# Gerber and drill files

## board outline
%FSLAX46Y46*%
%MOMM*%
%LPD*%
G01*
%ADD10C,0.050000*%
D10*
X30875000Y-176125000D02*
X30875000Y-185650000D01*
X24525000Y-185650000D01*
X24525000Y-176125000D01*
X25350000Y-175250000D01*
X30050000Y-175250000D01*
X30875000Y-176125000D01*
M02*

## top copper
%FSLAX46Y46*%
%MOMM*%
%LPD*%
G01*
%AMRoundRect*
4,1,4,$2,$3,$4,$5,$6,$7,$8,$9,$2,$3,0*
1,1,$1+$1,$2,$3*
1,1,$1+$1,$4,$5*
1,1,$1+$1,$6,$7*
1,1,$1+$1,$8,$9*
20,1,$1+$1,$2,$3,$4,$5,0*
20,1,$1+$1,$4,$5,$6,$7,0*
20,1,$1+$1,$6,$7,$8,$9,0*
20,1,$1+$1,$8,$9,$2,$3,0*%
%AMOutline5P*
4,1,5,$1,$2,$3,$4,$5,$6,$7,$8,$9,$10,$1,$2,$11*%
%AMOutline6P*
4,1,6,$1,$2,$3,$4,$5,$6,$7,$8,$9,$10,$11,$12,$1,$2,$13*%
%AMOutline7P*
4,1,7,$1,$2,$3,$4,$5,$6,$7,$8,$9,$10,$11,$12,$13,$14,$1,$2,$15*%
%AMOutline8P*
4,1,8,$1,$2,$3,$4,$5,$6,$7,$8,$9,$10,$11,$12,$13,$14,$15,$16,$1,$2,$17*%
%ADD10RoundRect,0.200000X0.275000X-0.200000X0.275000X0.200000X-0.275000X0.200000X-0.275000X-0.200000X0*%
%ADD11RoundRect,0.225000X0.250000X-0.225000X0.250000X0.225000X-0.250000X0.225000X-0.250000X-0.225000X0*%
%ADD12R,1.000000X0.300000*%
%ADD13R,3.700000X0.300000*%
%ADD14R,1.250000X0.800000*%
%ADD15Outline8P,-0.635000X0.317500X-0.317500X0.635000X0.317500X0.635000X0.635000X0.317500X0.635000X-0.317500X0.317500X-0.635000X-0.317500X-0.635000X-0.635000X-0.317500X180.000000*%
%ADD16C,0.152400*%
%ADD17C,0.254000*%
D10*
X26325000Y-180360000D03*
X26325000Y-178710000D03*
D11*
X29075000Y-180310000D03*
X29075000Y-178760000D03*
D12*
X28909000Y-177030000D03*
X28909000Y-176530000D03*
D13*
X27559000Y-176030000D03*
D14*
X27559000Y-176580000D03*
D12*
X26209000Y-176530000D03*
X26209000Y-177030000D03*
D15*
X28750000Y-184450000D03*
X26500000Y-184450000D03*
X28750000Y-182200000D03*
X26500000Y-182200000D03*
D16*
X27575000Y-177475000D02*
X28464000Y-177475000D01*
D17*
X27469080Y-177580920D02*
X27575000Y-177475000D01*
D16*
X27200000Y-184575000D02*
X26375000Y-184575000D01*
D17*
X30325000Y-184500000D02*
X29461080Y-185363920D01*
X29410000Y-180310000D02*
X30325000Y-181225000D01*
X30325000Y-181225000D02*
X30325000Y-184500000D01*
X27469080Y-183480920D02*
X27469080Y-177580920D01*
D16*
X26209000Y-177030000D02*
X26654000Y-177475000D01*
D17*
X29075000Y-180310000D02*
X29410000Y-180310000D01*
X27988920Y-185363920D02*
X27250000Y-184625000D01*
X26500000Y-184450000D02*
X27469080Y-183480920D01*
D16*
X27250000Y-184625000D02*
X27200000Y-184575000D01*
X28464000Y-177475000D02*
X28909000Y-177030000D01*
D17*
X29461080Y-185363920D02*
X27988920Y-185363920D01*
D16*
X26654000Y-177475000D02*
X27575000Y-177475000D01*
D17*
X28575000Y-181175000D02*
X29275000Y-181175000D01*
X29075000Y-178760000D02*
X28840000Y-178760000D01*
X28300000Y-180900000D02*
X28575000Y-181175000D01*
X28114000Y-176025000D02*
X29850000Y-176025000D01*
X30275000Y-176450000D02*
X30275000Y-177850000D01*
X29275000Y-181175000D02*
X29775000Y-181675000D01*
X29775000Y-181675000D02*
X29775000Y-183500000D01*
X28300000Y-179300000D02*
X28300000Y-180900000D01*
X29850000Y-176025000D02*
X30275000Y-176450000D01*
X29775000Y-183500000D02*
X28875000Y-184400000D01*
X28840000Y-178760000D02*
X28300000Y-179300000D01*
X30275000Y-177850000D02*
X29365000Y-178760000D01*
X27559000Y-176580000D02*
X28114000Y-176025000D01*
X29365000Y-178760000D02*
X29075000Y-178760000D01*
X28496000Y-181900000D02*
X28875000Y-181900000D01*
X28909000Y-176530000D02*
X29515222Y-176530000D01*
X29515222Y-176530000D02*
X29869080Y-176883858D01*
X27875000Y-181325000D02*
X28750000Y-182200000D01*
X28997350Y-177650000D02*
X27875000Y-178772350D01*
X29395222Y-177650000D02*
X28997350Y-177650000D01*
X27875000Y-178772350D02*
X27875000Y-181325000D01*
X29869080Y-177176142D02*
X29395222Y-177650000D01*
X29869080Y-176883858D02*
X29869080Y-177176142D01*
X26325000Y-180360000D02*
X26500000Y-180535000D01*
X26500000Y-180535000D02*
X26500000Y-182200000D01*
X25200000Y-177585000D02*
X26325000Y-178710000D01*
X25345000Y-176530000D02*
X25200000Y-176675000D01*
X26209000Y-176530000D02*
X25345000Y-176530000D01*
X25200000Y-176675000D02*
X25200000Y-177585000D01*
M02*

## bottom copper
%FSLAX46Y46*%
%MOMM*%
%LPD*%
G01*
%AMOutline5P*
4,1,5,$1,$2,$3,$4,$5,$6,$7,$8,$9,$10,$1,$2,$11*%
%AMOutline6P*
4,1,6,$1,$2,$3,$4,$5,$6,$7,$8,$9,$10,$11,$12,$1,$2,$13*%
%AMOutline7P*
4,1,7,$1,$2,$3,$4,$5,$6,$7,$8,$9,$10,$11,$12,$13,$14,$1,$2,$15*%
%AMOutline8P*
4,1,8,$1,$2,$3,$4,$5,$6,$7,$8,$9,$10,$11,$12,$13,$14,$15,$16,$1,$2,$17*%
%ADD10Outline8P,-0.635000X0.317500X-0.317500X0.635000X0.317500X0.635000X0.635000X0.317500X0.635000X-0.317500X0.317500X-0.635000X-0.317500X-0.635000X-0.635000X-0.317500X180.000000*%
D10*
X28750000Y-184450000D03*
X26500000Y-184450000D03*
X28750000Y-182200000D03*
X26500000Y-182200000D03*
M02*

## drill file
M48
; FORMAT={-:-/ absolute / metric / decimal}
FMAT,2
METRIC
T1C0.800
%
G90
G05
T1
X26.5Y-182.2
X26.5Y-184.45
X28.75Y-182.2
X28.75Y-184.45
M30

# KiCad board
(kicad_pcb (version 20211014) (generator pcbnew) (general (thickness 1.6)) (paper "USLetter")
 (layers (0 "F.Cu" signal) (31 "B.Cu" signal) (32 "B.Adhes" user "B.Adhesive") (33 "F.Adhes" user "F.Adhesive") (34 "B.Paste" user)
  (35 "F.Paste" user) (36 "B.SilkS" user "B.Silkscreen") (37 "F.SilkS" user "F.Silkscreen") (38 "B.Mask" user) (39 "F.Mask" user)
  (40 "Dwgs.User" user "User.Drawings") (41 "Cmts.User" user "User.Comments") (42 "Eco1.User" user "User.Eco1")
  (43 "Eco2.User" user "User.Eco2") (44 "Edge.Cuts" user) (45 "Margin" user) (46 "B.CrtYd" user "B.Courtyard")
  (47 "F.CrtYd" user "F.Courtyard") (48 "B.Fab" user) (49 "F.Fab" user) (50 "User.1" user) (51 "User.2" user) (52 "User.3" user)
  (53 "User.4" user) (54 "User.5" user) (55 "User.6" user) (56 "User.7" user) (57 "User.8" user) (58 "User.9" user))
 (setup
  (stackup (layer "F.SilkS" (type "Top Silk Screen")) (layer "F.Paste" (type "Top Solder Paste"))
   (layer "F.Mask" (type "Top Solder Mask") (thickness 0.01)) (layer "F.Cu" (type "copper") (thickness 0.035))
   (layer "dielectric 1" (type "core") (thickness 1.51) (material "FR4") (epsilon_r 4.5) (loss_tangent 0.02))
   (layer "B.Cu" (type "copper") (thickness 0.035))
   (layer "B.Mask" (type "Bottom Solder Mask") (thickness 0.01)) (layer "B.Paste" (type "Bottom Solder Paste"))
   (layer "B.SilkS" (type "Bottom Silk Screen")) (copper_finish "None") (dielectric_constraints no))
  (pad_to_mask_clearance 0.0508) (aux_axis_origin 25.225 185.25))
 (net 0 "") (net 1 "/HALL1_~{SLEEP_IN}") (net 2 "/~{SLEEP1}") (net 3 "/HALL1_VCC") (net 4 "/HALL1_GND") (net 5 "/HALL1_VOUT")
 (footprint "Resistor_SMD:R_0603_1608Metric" (layer "F.Cu") (at 26.325 179.535 90)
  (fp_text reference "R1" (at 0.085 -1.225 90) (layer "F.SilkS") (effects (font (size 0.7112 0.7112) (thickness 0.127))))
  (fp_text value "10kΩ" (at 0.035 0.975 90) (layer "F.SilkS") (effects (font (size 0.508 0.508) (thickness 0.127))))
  (pad "1" smd roundrect (at -0.825 0 90) (size 0.8 0.95) (layers "F.Cu" "F.Paste" "F.Mask") (roundrect_rratio 0.25)
   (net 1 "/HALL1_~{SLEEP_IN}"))
  (pad "2" smd roundrect (at 0.825 0 90) (size 0.8 0.95) (layers "F.Cu" "F.Paste" "F.Mask") (roundrect_rratio 0.25) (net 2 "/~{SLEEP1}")))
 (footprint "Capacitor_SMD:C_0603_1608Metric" (layer "F.Cu") (at 29.075 179.535 90)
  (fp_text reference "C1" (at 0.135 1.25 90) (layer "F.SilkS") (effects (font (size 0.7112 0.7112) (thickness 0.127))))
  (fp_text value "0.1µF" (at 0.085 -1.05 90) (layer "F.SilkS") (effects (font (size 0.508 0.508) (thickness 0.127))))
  (pad "1" smd roundrect (at -0.775 0 90) (size 0.9 0.95) (layers "F.Cu" "F.Paste" "F.Mask") (roundrect_rratio 0.25) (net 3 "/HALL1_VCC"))
  (pad "2" smd roundrect (at 0.775 0 90) (size 0.9 0.95) (layers "F.Cu" "F.Paste" "F.Mask") (roundrect_rratio 0.25) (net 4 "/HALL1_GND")))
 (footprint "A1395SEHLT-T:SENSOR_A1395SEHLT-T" (layer "F.Cu") (at 27.559 176.53 180)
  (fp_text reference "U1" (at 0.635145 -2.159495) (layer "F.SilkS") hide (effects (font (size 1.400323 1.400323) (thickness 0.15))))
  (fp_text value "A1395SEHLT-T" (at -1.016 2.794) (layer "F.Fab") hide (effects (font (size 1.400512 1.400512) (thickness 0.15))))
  (pad "1" smd rect locked (at -1.35 -0.5 180) (size 1 0.3) (layers "F.Cu" "F.Paste" "F.Mask") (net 3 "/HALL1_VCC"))
  (pad "2" smd rect locked (at -1.35 0 180) (size 1 0.3) (layers "F.Cu" "F.Paste" "F.Mask") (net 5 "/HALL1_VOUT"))
  (pad "3" smd rect locked (at 0 0.5 90) (size 0.3 3.7) (layers "F.Cu" "F.Paste" "F.Mask") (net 4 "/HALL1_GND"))
  (pad "4" smd rect locked (at 0 -0.05 180) (size 1.25 0.8) (layers "F.Cu" "F.Mask") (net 4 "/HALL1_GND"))
  (pad "5" smd rect locked (at 1.35 0 180) (size 1 0.3) (layers "F.Cu" "F.Paste" "F.Mask") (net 2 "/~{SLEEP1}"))
  (pad "6" smd rect locked (at 1.35 -0.5 180) (size 1 0.3) (layers "F.Cu" "F.Paste" "F.Mask") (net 3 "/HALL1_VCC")))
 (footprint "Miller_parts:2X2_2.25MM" (layer "F.Cu") (at 27.625 183.325 180)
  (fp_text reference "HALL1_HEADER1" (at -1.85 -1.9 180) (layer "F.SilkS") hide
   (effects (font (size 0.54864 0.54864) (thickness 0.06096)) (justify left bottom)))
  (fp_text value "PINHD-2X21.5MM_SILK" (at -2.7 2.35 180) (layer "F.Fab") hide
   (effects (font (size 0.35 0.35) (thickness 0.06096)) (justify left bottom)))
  (pad "P$1" thru_hole roundrect (at -1.125 -1.125 180) (size 1.27 1.27) (drill 0.8) (layers *.Cu *.Mask) (roundrect_rratio 0.25)
   (chamfer_ratio 0.25) (chamfer top_left top_right bottom_left bottom_right) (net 4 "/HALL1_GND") (solder_mask_margin 0.0762))
  (pad "P$2" thru_hole roundrect (at 1.125 -1.125 180) (size 1.27 1.27) (drill 0.8) (layers *.Cu *.Mask) (roundrect_rratio 0.25)
   (chamfer_ratio 0.25) (chamfer top_left top_right bottom_left bottom_right) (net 3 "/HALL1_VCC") (solder_mask_margin 0.0762))
  (pad "P$3" thru_hole roundrect (at -1.125 1.125 180) (size 1.27 1.27) (drill 0.8) (layers *.Cu *.Mask) (roundrect_rratio 0.25)
   (chamfer_ratio 0.25) (chamfer top_left top_right bottom_left bottom_right) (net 5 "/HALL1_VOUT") (solder_mask_margin 0.0762))
  (pad "P$4" thru_hole roundrect (at 1.125 1.125 180) (size 1.27 1.27) (drill 0.8) (layers *.Cu *.Mask) (roundrect_rratio 0.25)
   (chamfer_ratio 0.25) (chamfer top_left top_right bottom_left bottom_right) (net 1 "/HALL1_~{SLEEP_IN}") (solder_mask_margin 0.0762)))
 (gr_poly
  (pts (xy 30.875 176.125) (xy 30.875 185.65) (xy 24.525 185.65) (xy 24.525 176.125) (xy 25.35 175.25) (xy 30.05 175.25))
  (layer "Edge.Cuts") (width 0.05) (fill none))
 (segment (start 27.575 177.475) (end 28.464 177.475) (width 0.1524) (layer "F.Cu") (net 3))
 (segment (start 27.46908 177.58092) (end 27.575 177.475) (width 0.254) (layer "F.Cu") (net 3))
 (segment (start 27.2 184.575) (end 26.375 184.575) (width 0.1524) (layer "F.Cu") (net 3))
 (segment (start 30.325 184.5) (end 29.46108 185.36392) (width 0.254) (layer "F.Cu") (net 3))
 (segment (start 29.41 180.31) (end 30.325 181.225) (width 0.254) (layer "F.Cu") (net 3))
 (segment (start 30.325 181.225) (end 30.325 184.5) (width 0.254) (layer "F.Cu") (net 3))
 (segment (start 27.46908 183.48092) (end 27.46908 177.58092) (width 0.254) (layer "F.Cu") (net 3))
 (segment (start 26.209 177.03) (end 26.654 177.475) (width 0.1524) (layer "F.Cu") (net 3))
 (segment (start 29.075 180.31) (end 29.41 180.31) (width 0.254) (layer "F.Cu") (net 3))
 (segment (start 27.98892 185.36392) (end 27.25 184.625) (width 0.254) (layer "F.Cu") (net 3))
 (segment (start 26.5 184.45) (end 27.46908 183.48092) (width 0.254) (layer "F.Cu") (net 3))
 (segment (start 27.25 184.625) (end 27.2 184.575) (width 0.1524) (layer "F.Cu") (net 3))
 (segment (start 28.464 177.475) (end 28.909 177.03) (width 0.1524) (layer "F.Cu") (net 3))
 (segment (start 29.46108 185.36392) (end 27.98892 185.36392) (width 0.254) (layer "F.Cu") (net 3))
 (segment (start 26.654 177.475) (end 27.575 177.475) (width 0.1524) (layer "F.Cu") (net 3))
 (segment (start 28.575 181.175) (end 29.275 181.175) (width 0.254) (layer "F.Cu") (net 4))
 (segment (start 29.075 178.76) (end 28.84 178.76) (width 0.254) (layer "F.Cu") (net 4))
 (segment (start 28.3 180.9) (end 28.575 181.175) (width 0.254) (layer "F.Cu") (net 4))
 (segment (start 28.114 176.025) (end 29.85 176.025) (width 0.254) (layer "F.Cu") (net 4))
 (segment (start 30.275 176.45) (end 30.275 177.85) (width 0.254) (layer "F.Cu") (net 4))
 (segment (start 29.275 181.175) (end 29.775 181.675) (width 0.254) (layer "F.Cu") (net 4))
 (segment (start 29.775 181.675) (end 29.775 183.5) (width 0.254) (layer "F.Cu") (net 4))
 (segment (start 28.3 179.3) (end 28.3 180.9) (width 0.254) (layer "F.Cu") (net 4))
 (segment (start 29.85 176.025) (end 30.275 176.45) (width 0.254) (layer "F.Cu") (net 4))
 (segment (start 29.775 183.5) (end 28.875 184.4) (width 0.254) (layer "F.Cu") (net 4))
 (segment (start 28.84 178.76) (end 28.3 179.3) (width 0.254) (layer "F.Cu") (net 4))
 (segment (start 30.275 177.85) (end 29.365 178.76) (width 0.254) (layer "F.Cu") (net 4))
 (segment (start 27.559 176.58) (end 28.114 176.025) (width 0.254) (layer "F.Cu") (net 4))
 (segment (start 29.365 178.76) (end 29.075 178.76) (width 0.254) (layer "F.Cu") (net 4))
 (segment (start 28.496 181.9) (end 28.875 181.9) (width 0.254) (layer "F.Cu") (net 5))
 (segment (start 28.909 176.53) (end 29.515222 176.53) (width 0.254) (layer "F.Cu") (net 5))
 (segment (start 29.515222 176.53) (end 29.86908 176.883858) (width 0.254) (layer "F.Cu") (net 5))
 (segment (start 27.875 181.325) (end 28.75 182.2) (width 0.254) (layer "F.Cu") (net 5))
 (segment (start 28.99735 177.65) (end 27.875 178.77235) (width 0.254) (layer "F.Cu") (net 5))
 (segment (start 29.395222 177.65) (end 28.99735 177.65) (width 0.254) (layer "F.Cu") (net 5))
 (segment (start 27.875 178.77235) (end 27.875 181.325) (width 0.254) (layer "F.Cu") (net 5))
 (segment (start 29.86908 177.176142) (end 29.395222 177.65) (width 0.254) (layer "F.Cu") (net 5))
 (segment (start 29.86908 176.883858) (end 29.86908 177.176142) (width 0.254) (layer "F.Cu") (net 5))
 (segment (start 26.325 180.36) (end 26.5 180.535) (width 0.254) (layer "F.Cu") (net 1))
 (segment (start 26.5 180.535) (end 26.5 182.2) (width 0.254) (layer "F.Cu") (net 1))
 (segment (start 25.2 177.585) (end 26.325 178.71) (width 0.254) (layer "F.Cu") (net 2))
 (segment (start 25.345 176.53) (end 25.2 176.675) (width 0.254) (layer "F.Cu") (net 2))
 (segment (start 26.209 176.53) (end 25.345 176.53) (width 0.254) (layer "F.Cu") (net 2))
 (segment (start 25.2 176.675) (end 25.2 177.585) (width 0.254) (layer "F.Cu") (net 2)))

